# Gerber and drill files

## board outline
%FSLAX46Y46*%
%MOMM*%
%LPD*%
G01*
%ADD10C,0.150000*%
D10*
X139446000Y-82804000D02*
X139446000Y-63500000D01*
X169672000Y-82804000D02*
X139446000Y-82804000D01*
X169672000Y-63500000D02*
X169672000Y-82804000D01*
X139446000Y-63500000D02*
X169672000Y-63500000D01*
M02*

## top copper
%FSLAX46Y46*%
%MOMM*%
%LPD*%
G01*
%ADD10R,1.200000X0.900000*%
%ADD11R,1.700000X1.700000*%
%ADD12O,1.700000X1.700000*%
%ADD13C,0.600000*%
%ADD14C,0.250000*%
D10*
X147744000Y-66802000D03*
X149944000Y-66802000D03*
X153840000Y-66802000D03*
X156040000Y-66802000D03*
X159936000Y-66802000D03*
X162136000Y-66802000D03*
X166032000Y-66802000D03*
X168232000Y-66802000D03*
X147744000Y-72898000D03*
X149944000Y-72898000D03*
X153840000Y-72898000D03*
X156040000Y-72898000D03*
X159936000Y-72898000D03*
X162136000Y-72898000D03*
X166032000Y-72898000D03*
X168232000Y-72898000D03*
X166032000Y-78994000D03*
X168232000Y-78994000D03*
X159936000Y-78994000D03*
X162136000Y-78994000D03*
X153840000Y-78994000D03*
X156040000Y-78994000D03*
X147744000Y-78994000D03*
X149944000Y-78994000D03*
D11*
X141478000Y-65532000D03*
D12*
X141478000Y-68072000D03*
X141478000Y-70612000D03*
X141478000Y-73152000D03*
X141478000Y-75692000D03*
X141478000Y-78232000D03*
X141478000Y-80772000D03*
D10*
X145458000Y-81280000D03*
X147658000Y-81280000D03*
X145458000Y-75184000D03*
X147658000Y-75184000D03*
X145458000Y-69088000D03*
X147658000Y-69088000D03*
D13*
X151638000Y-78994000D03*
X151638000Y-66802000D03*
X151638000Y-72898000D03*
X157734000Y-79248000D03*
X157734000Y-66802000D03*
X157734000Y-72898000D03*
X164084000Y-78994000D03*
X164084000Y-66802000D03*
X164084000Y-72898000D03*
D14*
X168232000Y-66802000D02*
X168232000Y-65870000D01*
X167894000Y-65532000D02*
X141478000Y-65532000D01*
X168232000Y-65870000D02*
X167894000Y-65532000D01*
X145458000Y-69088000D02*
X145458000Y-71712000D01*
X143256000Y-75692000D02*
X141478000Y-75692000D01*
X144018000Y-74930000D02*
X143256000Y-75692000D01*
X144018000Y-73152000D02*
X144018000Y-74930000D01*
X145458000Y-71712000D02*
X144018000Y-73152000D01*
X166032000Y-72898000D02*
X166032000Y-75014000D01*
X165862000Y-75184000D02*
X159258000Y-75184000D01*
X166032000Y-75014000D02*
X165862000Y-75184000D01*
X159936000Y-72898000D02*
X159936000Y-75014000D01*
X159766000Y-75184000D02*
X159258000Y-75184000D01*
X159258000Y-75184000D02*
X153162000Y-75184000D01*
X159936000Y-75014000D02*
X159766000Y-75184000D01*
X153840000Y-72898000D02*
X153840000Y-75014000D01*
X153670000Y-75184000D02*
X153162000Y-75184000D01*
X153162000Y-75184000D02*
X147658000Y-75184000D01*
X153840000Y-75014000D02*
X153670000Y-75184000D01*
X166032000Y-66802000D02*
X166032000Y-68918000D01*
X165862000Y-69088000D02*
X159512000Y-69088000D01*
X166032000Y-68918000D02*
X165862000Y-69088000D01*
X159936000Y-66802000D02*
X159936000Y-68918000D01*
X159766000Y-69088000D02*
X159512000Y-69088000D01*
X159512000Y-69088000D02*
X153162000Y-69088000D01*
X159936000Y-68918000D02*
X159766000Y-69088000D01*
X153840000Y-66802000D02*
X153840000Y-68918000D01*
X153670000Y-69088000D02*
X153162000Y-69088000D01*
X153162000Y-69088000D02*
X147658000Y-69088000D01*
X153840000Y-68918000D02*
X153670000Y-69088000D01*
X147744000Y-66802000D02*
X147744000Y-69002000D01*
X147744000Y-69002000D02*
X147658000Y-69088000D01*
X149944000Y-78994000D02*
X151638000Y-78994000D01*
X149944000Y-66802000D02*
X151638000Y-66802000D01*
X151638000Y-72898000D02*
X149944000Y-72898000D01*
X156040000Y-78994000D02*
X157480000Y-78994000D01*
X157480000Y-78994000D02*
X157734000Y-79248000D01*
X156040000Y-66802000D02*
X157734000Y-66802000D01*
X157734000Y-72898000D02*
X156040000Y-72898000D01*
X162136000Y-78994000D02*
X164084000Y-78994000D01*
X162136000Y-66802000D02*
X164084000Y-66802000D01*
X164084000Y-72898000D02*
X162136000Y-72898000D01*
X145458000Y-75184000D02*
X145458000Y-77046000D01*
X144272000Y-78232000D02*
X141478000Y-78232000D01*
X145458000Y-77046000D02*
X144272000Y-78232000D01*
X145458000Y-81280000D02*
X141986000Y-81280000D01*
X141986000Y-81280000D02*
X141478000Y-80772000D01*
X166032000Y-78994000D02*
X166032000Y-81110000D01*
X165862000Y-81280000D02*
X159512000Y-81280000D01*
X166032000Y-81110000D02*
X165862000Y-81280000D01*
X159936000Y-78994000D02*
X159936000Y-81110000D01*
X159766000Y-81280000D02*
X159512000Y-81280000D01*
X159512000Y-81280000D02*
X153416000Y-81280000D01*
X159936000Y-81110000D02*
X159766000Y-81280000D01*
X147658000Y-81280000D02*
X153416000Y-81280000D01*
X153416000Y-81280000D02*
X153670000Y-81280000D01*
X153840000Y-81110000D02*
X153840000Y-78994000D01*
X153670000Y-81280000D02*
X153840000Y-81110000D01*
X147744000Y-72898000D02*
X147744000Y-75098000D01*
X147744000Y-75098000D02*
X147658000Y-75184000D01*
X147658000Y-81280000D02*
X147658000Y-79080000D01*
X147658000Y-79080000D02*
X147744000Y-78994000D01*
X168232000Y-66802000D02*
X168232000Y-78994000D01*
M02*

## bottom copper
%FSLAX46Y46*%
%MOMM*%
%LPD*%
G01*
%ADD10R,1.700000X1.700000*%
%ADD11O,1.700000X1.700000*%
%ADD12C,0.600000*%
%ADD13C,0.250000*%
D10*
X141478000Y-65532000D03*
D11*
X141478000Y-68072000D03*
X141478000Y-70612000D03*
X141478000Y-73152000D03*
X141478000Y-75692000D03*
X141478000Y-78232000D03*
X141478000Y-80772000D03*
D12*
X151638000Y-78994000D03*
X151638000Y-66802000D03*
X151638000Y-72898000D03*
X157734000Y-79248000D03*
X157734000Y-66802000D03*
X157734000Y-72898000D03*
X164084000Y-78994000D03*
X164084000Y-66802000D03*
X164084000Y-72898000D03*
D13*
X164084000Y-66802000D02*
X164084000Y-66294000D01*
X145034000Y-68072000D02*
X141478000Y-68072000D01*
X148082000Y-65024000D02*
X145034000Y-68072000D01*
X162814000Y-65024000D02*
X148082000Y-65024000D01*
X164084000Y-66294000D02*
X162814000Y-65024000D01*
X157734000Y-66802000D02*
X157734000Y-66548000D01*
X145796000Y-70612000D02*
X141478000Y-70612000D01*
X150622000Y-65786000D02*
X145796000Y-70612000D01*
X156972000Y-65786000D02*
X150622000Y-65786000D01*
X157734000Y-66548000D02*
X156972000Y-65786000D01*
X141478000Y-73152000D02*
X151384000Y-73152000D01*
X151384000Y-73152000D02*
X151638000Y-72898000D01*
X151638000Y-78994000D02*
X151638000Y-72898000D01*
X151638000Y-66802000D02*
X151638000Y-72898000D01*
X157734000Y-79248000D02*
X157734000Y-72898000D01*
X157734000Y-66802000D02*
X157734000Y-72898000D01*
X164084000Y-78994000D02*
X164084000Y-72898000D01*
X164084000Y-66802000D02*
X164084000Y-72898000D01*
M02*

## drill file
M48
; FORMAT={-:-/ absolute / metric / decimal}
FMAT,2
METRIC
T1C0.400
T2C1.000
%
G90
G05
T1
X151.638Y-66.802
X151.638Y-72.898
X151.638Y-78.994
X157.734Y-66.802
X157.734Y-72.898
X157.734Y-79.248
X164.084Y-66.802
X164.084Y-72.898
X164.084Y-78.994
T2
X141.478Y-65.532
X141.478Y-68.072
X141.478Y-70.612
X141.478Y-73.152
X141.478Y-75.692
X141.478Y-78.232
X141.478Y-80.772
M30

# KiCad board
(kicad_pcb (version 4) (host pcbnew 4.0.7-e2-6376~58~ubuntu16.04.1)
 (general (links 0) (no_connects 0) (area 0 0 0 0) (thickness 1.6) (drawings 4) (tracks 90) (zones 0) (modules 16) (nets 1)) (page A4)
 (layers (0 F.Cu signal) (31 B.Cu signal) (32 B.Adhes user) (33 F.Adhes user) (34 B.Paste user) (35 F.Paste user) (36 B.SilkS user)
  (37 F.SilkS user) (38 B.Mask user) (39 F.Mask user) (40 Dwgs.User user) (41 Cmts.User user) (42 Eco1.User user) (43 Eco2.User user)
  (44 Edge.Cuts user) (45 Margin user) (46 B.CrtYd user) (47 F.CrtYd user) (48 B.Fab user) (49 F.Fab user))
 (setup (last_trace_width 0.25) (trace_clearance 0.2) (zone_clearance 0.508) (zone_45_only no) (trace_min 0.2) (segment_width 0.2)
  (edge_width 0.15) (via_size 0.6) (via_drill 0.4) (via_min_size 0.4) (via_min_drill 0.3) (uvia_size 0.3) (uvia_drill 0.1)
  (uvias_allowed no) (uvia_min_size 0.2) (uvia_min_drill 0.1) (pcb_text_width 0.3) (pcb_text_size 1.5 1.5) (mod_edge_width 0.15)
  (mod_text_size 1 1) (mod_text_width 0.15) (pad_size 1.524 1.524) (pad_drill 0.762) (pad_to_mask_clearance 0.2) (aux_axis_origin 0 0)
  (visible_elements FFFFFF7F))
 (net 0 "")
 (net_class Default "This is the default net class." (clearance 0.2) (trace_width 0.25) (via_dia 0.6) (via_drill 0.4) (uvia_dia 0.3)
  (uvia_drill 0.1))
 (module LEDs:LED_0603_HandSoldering (layer F.Cu) (at 148.844 66.802)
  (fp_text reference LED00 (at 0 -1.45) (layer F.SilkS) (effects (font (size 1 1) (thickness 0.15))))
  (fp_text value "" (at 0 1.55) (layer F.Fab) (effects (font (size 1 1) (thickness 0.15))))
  (pad 1 smd rect (at -1.1 0) (size 1.2 0.9) (layers F.Cu F.Paste F.Mask))
  (pad 2 smd rect (at 1.1 0) (size 1.2 0.9) (layers F.Cu F.Paste F.Mask)))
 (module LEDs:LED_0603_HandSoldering (layer F.Cu) (at 154.94 66.802)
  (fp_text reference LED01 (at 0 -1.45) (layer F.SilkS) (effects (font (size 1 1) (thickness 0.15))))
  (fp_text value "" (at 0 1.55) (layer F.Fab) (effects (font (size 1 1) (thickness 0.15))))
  (pad 1 smd rect (at -1.1 0) (size 1.2 0.9) (layers F.Cu F.Paste F.Mask))
  (pad 2 smd rect (at 1.1 0) (size 1.2 0.9) (layers F.Cu F.Paste F.Mask)))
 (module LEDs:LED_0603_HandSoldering (layer F.Cu) (at 161.036 66.802)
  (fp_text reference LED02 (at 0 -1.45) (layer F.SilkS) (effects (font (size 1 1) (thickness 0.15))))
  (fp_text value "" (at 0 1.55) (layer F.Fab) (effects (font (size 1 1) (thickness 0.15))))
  (pad 1 smd rect (at -1.1 0) (size 1.2 0.9) (layers F.Cu F.Paste F.Mask))
  (pad 2 smd rect (at 1.1 0) (size 1.2 0.9) (layers F.Cu F.Paste F.Mask)))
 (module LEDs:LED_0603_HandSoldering (layer F.Cu) (at 167.132 66.802)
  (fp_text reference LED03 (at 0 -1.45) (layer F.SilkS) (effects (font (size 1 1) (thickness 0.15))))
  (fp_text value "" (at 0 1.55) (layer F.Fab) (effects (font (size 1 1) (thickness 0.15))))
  (pad 1 smd rect (at -1.1 0) (size 1.2 0.9) (layers F.Cu F.Paste F.Mask))
  (pad 2 smd rect (at 1.1 0) (size 1.2 0.9) (layers F.Cu F.Paste F.Mask)))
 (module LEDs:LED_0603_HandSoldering (layer F.Cu) (at 148.844 72.898)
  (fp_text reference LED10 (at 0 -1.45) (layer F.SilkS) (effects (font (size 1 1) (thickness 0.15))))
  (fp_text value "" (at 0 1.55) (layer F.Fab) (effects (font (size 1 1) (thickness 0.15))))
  (pad 1 smd rect (at -1.1 0) (size 1.2 0.9) (layers F.Cu F.Paste F.Mask))
  (pad 2 smd rect (at 1.1 0) (size 1.2 0.9) (layers F.Cu F.Paste F.Mask)))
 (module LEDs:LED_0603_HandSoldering (layer F.Cu) (at 154.94 72.898)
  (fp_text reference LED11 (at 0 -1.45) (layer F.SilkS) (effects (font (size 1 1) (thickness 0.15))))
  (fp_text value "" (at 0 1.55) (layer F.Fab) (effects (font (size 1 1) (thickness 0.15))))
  (pad 1 smd rect (at -1.1 0) (size 1.2 0.9) (layers F.Cu F.Paste F.Mask))
  (pad 2 smd rect (at 1.1 0) (size 1.2 0.9) (layers F.Cu F.Paste F.Mask)))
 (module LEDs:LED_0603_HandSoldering (layer F.Cu) (at 161.036 72.898)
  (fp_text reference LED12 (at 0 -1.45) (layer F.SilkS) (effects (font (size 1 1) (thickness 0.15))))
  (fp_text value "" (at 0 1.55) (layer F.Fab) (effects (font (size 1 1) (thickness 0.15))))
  (pad 1 smd rect (at -1.1 0) (size 1.2 0.9) (layers F.Cu F.Paste F.Mask))
  (pad 2 smd rect (at 1.1 0) (size 1.2 0.9) (layers F.Cu F.Paste F.Mask)))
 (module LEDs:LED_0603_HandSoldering (layer F.Cu) (at 167.132 72.898)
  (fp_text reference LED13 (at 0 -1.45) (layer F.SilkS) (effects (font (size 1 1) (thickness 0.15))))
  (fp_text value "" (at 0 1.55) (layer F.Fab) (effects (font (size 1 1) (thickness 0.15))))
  (pad 1 smd rect (at -1.1 0) (size 1.2 0.9) (layers F.Cu F.Paste F.Mask))
  (pad 2 smd rect (at 1.1 0) (size 1.2 0.9) (layers F.Cu F.Paste F.Mask)))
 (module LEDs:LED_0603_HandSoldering (layer F.Cu) (at 167.132 78.994)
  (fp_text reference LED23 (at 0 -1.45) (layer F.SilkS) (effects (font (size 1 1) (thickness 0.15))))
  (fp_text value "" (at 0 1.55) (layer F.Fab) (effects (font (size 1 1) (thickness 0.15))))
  (pad 1 smd rect (at -1.1 0) (size 1.2 0.9) (layers F.Cu F.Paste F.Mask))
  (pad 2 smd rect (at 1.1 0) (size 1.2 0.9) (layers F.Cu F.Paste F.Mask)))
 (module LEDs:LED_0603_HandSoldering (layer F.Cu) (at 161.036 78.994)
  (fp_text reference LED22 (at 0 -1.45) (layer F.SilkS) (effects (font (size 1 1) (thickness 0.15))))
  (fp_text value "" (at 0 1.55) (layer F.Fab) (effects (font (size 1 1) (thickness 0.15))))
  (pad 1 smd rect (at -1.1 0) (size 1.2 0.9) (layers F.Cu F.Paste F.Mask))
  (pad 2 smd rect (at 1.1 0) (size 1.2 0.9) (layers F.Cu F.Paste F.Mask)))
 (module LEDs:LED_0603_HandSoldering (layer F.Cu) (at 154.94 78.994)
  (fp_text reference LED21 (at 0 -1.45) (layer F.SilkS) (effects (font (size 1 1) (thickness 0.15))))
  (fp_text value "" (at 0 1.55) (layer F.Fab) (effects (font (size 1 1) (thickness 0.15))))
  (pad 1 smd rect (at -1.1 0) (size 1.2 0.9) (layers F.Cu F.Paste F.Mask))
  (pad 2 smd rect (at 1.1 0) (size 1.2 0.9) (layers F.Cu F.Paste F.Mask)))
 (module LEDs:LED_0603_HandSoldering (layer F.Cu) (at 148.844 78.994)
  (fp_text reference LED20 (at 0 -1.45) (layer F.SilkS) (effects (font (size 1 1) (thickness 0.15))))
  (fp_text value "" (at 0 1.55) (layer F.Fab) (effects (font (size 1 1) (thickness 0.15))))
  (pad 1 smd rect (at -1.1 0) (size 1.2 0.9) (layers F.Cu F.Paste F.Mask))
  (pad 2 smd rect (at 1.1 0) (size 1.2 0.9) (layers F.Cu F.Paste F.Mask)))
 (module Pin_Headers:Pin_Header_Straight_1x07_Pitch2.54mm (layer F.Cu) (at 141.478 65.532)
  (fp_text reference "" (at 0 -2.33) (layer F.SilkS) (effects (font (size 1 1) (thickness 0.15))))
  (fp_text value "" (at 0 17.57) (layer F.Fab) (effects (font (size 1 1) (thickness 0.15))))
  (pad 1 thru_hole rect (at 0 0) (size 1.7 1.7) (drill 1) (layers *.Cu *.Mask))
  (pad 2 thru_hole oval (at 0 2.54) (size 1.7 1.7) (drill 1) (layers *.Cu *.Mask))
  (pad 3 thru_hole oval (at 0 5.08) (size 1.7 1.7) (drill 1) (layers *.Cu *.Mask))
  (pad 4 thru_hole oval (at 0 7.62) (size 1.7 1.7) (drill 1) (layers *.Cu *.Mask))
  (pad 5 thru_hole oval (at 0 10.16) (size 1.7 1.7) (drill 1) (layers *.Cu *.Mask))
  (pad 6 thru_hole oval (at 0 12.7) (size 1.7 1.7) (drill 1) (layers *.Cu *.Mask))
  (pad 7 thru_hole oval (at 0 15.24) (size 1.7 1.7) (drill 1) (layers *.Cu *.Mask)))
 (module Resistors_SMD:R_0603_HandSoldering (layer F.Cu) (at 146.558 81.28)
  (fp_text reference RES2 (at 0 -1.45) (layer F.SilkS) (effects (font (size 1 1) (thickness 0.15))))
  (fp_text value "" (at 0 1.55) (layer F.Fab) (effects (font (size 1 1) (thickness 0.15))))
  (pad 1 smd rect (at -1.1 0) (size 1.2 0.9) (layers F.Cu F.Paste F.Mask))
  (pad 2 smd rect (at 1.1 0) (size 1.2 0.9) (layers F.Cu F.Paste F.Mask)))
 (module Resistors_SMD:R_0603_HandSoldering (layer F.Cu) (at 146.558 75.184)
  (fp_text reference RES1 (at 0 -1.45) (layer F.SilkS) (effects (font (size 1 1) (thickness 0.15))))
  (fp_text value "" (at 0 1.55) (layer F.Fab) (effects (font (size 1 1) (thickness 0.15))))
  (pad 1 smd rect (at -1.1 0) (size 1.2 0.9) (layers F.Cu F.Paste F.Mask))
  (pad 2 smd rect (at 1.1 0) (size 1.2 0.9) (layers F.Cu F.Paste F.Mask)))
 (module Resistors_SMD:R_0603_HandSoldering (layer F.Cu) (at 146.558 69.088)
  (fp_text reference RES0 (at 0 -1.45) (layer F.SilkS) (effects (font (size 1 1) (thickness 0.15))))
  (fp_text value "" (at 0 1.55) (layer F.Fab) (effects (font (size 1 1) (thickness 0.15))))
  (pad 1 smd rect (at -1.1 0) (size 1.2 0.9) (layers F.Cu F.Paste F.Mask))
  (pad 2 smd rect (at 1.1 0) (size 1.2 0.9) (layers F.Cu F.Paste F.Mask)))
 (gr_line (start 139.446 82.804) (end 139.446 63.5) (angle 90) (layer Edge.Cuts) (width 0.15))
 (gr_line (start 169.672 82.804) (end 139.446 82.804) (angle 90) (layer Edge.Cuts) (width 0.15))
 (gr_line (start 169.672 63.5) (end 169.672 82.804) (angle 90) (layer Edge.Cuts) (width 0.15))
 (gr_line (start 139.446 63.5) (end 169.672 63.5) (angle 90) (layer Edge.Cuts) (width 0.15))
 (segment (start 164.084 66.802) (end 164.084 66.294) (width 0.25) (layer B.Cu) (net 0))
 (segment (start 145.034 68.072) (end 141.478 68.072) (width 0.25) (layer B.Cu) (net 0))
 (segment (start 148.082 65.024) (end 145.034 68.072) (width 0.25) (layer B.Cu) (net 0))
 (segment (start 162.814 65.024) (end 148.082 65.024) (width 0.25) (layer B.Cu) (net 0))
 (segment (start 164.084 66.294) (end 162.814 65.024) (width 0.25) (layer B.Cu) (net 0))
 (segment (start 168.232 66.802) (end 168.232 65.87) (width 0.25) (layer F.Cu) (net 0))
 (segment (start 167.894 65.532) (end 141.478 65.532) (width 0.25) (layer F.Cu) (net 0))
 (segment (start 168.232 65.87) (end 167.894 65.532) (width 0.25) (layer F.Cu) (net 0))
 (segment (start 157.734 66.802) (end 157.734 66.548) (width 0.25) (layer B.Cu) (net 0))
 (segment (start 145.796 70.612) (end 141.478 70.612) (width 0.25) (layer B.Cu) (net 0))
 (segment (start 150.622 65.786) (end 145.796 70.612) (width 0.25) (layer B.Cu) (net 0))
 (segment (start 156.972 65.786) (end 150.622 65.786) (width 0.25) (layer B.Cu) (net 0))
 (segment (start 157.734 66.548) (end 156.972 65.786) (width 0.25) (layer B.Cu) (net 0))
 (segment (start 141.478 73.152) (end 151.384 73.152) (width 0.25) (layer B.Cu) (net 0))
 (segment (start 151.384 73.152) (end 151.638 72.898) (width 0.25) (layer B.Cu) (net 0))
 (segment (start 145.458 69.088) (end 145.458 71.712) (width 0.25) (layer F.Cu) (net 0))
 (segment (start 143.256 75.692) (end 141.478 75.692) (width 0.25) (layer F.Cu) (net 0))
 (segment (start 144.018 74.93) (end 143.256 75.692) (width 0.25) (layer F.Cu) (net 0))
 (segment (start 144.018 73.152) (end 144.018 74.93) (width 0.25) (layer F.Cu) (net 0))
 (segment (start 145.458 71.712) (end 144.018 73.152) (width 0.25) (layer F.Cu) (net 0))
 (segment (start 166.032 72.898) (end 166.032 75.014) (width 0.25) (layer F.Cu) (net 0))
 (segment (start 165.862 75.184) (end 159.258 75.184) (width 0.25) (layer F.Cu) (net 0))
 (segment (start 166.032 75.014) (end 165.862 75.184) (width 0.25) (layer F.Cu) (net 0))
 (segment (start 159.936 72.898) (end 159.936 75.014) (width 0.25) (layer F.Cu) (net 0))
 (segment (start 159.766 75.184) (end 159.258 75.184) (width 0.25) (layer F.Cu) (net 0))
 (segment (start 159.258 75.184) (end 153.162 75.184) (width 0.25) (layer F.Cu) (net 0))
 (segment (start 159.936 75.014) (end 159.766 75.184) (width 0.25) (layer F.Cu) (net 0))
 (segment (start 153.84 72.898) (end 153.84 75.014) (width 0.25) (layer F.Cu) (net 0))
 (segment (start 153.67 75.184) (end 153.162 75.184) (width 0.25) (layer F.Cu) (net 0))
 (segment (start 153.162 75.184) (end 147.658 75.184) (width 0.25) (layer F.Cu) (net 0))
 (segment (start 153.84 75.014) (end 153.67 75.184) (width 0.25) (layer F.Cu) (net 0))
 (segment (start 166.032 66.802) (end 166.032 68.918) (width 0.25) (layer F.Cu) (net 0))
 (segment (start 165.862 69.088) (end 159.512 69.088) (width 0.25) (layer F.Cu) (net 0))
 (segment (start 166.032 68.918) (end 165.862 69.088) (width 0.25) (layer F.Cu) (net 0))
 (segment (start 159.936 66.802) (end 159.936 68.918) (width 0.25) (layer F.Cu) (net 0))
 (segment (start 159.766 69.088) (end 159.512 69.088) (width 0.25) (layer F.Cu) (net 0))
 (segment (start 159.512 69.088) (end 153.162 69.088) (width 0.25) (layer F.Cu) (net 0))
 (segment (start 159.936 68.918) (end 159.766 69.088) (width 0.25) (layer F.Cu) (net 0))
 (segment (start 153.84 66.802) (end 153.84 68.918) (width 0.25) (layer F.Cu) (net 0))
 (segment (start 153.67 69.088) (end 153.162 69.088) (width 0.25) (layer F.Cu) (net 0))
 (segment (start 153.162 69.088) (end 147.658 69.088) (width 0.25) (layer F.Cu) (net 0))
 (segment (start 153.84 68.918) (end 153.67 69.088) (width 0.25) (layer F.Cu) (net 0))
 (segment (start 147.744 66.802) (end 147.744 69.002) (width 0.25) (layer F.Cu) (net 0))
 (segment (start 147.744 69.002) (end 147.658 69.088) (width 0.25) (layer F.Cu) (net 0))
 (segment (start 149.944 78.994) (end 151.638 78.994) (width 0.25) (layer F.Cu) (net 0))
 (segment (start 151.638 78.994) (end 151.638 72.898) (width 0.25) (layer B.Cu) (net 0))
 (via (at 151.638 78.994) (size 0.6) (drill 0.4) (layers F.Cu B.Cu) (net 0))
 (segment (start 149.944 66.802) (end 151.638 66.802) (width 0.25) (layer F.Cu) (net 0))
 (via (at 151.638 66.802) (size 0.6) (drill 0.4) (layers F.Cu B.Cu) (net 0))
 (segment (start 151.638 66.802) (end 151.638 72.898) (width 0.25) (layer B.Cu) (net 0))
 (segment (start 151.638 72.898) (end 149.944 72.898) (width 0.25) (layer F.Cu) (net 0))
 (via (at 151.638 72.898) (size 0.6) (drill 0.4) (layers F.Cu B.Cu) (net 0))
 (segment (start 156.04 78.994) (end 157.48 78.994) (width 0.25) (layer F.Cu) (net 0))
 (segment (start 157.734 79.248) (end 157.734 72.898) (width 0.25) (layer B.Cu) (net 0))
 (via (at 157.734 79.248) (size 0.6) (drill 0.4) (layers F.Cu B.Cu) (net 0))
 (segment (start 157.48 78.994) (end 157.734 79.248) (width 0.25) (layer F.Cu) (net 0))
 (segment (start 156.04 66.802) (end 157.734 66.802) (width 0.25) (layer F.Cu) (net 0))
 (via (at 157.734 66.802) (size 0.6) (drill 0.4) (layers F.Cu B.Cu) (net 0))
 (segment (start 157.734 66.802) (end 157.734 72.898) (width 0.25) (layer B.Cu) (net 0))
 (segment (start 157.734 72.898) (end 156.04 72.898) (width 0.25) (layer F.Cu) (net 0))
 (via (at 157.734 72.898) (size 0.6) (drill 0.4) (layers F.Cu B.Cu) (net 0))
 (segment (start 162.136 78.994) (end 164.084 78.994) (width 0.25) (layer F.Cu) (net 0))
 (segment (start 164.084 78.994) (end 164.084 72.898) (width 0.25) (layer B.Cu) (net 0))
 (via (at 164.084 78.994) (size 0.6) (drill 0.4) (layers F.Cu B.Cu) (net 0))
 (segment (start 162.136 66.802) (end 164.084 66.802) (width 0.25) (layer F.Cu) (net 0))
 (via (at 164.084 66.802) (size 0.6) (drill 0.4) (layers F.Cu B.Cu) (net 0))
 (segment (start 164.084 66.802) (end 164.084 72.898) (width 0.25) (layer B.Cu) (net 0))
 (segment (start 164.084 72.898) (end 162.136 72.898) (width 0.25) (layer F.Cu) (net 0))
 (via (at 164.084 72.898) (size 0.6) (drill 0.4) (layers F.Cu B.Cu) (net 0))
 (segment (start 145.458 75.184) (end 145.458 77.046) (width 0.25) (layer F.Cu) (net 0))
 (segment (start 144.272 78.232) (end 141.478 78.232) (width 0.25) (layer F.Cu) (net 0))
 (segment (start 145.458 77.046) (end 144.272 78.232) (width 0.25) (layer F.Cu) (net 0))
 (segment (start 145.458 81.28) (end 141.986 81.28) (width 0.25) (layer F.Cu) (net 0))
 (segment (start 141.986 81.28) (end 141.478 80.772) (width 0.25) (layer F.Cu) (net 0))
 (segment (start 166.032 78.994) (end 166.032 81.11) (width 0.25) (layer F.Cu) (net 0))
 (segment (start 165.862 81.28) (end 159.512 81.28) (width 0.25) (layer F.Cu) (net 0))
 (segment (start 166.032 81.11) (end 165.862 81.28) (width 0.25) (layer F.Cu) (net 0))
 (segment (start 159.936 78.994) (end 159.936 81.11) (width 0.25) (layer F.Cu) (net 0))
 (segment (start 159.766 81.28) (end 159.512 81.28) (width 0.25) (layer F.Cu) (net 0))
 (segment (start 159.512 81.28) (end 153.416 81.28) (width 0.25) (layer F.Cu) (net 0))
 (segment (start 159.936 81.11) (end 159.766 81.28) (width 0.25) (layer F.Cu) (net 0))
 (segment (start 147.658 81.28) (end 153.416 81.28) (width 0.25) (layer F.Cu) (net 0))
 (segment (start 153.416 81.28) (end 153.67 81.28) (width 0.25) (layer F.Cu) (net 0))
 (segment (start 153.84 81.11) (end 153.84 78.994) (width 0.25) (layer F.Cu) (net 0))
 (segment (start 153.67 81.28) (end 153.84 81.11) (width 0.25) (layer F.Cu) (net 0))
 (segment (start 147.744 72.898) (end 147.744 75.098) (width 0.25) (layer F.Cu) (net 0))
 (segment (start 147.744 75.098) (end 147.658 75.184) (width 0.25) (layer F.Cu) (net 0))
 (segment (start 147.658 81.28) (end 147.658 79.08) (width 0.25) (layer F.Cu) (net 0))
 (segment (start 147.658 79.08) (end 147.744 78.994) (width 0.25) (layer F.Cu) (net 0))
 (segment (start 168.232 66.802) (end 168.232 78.994) (width 0.25) (layer F.Cu) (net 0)))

